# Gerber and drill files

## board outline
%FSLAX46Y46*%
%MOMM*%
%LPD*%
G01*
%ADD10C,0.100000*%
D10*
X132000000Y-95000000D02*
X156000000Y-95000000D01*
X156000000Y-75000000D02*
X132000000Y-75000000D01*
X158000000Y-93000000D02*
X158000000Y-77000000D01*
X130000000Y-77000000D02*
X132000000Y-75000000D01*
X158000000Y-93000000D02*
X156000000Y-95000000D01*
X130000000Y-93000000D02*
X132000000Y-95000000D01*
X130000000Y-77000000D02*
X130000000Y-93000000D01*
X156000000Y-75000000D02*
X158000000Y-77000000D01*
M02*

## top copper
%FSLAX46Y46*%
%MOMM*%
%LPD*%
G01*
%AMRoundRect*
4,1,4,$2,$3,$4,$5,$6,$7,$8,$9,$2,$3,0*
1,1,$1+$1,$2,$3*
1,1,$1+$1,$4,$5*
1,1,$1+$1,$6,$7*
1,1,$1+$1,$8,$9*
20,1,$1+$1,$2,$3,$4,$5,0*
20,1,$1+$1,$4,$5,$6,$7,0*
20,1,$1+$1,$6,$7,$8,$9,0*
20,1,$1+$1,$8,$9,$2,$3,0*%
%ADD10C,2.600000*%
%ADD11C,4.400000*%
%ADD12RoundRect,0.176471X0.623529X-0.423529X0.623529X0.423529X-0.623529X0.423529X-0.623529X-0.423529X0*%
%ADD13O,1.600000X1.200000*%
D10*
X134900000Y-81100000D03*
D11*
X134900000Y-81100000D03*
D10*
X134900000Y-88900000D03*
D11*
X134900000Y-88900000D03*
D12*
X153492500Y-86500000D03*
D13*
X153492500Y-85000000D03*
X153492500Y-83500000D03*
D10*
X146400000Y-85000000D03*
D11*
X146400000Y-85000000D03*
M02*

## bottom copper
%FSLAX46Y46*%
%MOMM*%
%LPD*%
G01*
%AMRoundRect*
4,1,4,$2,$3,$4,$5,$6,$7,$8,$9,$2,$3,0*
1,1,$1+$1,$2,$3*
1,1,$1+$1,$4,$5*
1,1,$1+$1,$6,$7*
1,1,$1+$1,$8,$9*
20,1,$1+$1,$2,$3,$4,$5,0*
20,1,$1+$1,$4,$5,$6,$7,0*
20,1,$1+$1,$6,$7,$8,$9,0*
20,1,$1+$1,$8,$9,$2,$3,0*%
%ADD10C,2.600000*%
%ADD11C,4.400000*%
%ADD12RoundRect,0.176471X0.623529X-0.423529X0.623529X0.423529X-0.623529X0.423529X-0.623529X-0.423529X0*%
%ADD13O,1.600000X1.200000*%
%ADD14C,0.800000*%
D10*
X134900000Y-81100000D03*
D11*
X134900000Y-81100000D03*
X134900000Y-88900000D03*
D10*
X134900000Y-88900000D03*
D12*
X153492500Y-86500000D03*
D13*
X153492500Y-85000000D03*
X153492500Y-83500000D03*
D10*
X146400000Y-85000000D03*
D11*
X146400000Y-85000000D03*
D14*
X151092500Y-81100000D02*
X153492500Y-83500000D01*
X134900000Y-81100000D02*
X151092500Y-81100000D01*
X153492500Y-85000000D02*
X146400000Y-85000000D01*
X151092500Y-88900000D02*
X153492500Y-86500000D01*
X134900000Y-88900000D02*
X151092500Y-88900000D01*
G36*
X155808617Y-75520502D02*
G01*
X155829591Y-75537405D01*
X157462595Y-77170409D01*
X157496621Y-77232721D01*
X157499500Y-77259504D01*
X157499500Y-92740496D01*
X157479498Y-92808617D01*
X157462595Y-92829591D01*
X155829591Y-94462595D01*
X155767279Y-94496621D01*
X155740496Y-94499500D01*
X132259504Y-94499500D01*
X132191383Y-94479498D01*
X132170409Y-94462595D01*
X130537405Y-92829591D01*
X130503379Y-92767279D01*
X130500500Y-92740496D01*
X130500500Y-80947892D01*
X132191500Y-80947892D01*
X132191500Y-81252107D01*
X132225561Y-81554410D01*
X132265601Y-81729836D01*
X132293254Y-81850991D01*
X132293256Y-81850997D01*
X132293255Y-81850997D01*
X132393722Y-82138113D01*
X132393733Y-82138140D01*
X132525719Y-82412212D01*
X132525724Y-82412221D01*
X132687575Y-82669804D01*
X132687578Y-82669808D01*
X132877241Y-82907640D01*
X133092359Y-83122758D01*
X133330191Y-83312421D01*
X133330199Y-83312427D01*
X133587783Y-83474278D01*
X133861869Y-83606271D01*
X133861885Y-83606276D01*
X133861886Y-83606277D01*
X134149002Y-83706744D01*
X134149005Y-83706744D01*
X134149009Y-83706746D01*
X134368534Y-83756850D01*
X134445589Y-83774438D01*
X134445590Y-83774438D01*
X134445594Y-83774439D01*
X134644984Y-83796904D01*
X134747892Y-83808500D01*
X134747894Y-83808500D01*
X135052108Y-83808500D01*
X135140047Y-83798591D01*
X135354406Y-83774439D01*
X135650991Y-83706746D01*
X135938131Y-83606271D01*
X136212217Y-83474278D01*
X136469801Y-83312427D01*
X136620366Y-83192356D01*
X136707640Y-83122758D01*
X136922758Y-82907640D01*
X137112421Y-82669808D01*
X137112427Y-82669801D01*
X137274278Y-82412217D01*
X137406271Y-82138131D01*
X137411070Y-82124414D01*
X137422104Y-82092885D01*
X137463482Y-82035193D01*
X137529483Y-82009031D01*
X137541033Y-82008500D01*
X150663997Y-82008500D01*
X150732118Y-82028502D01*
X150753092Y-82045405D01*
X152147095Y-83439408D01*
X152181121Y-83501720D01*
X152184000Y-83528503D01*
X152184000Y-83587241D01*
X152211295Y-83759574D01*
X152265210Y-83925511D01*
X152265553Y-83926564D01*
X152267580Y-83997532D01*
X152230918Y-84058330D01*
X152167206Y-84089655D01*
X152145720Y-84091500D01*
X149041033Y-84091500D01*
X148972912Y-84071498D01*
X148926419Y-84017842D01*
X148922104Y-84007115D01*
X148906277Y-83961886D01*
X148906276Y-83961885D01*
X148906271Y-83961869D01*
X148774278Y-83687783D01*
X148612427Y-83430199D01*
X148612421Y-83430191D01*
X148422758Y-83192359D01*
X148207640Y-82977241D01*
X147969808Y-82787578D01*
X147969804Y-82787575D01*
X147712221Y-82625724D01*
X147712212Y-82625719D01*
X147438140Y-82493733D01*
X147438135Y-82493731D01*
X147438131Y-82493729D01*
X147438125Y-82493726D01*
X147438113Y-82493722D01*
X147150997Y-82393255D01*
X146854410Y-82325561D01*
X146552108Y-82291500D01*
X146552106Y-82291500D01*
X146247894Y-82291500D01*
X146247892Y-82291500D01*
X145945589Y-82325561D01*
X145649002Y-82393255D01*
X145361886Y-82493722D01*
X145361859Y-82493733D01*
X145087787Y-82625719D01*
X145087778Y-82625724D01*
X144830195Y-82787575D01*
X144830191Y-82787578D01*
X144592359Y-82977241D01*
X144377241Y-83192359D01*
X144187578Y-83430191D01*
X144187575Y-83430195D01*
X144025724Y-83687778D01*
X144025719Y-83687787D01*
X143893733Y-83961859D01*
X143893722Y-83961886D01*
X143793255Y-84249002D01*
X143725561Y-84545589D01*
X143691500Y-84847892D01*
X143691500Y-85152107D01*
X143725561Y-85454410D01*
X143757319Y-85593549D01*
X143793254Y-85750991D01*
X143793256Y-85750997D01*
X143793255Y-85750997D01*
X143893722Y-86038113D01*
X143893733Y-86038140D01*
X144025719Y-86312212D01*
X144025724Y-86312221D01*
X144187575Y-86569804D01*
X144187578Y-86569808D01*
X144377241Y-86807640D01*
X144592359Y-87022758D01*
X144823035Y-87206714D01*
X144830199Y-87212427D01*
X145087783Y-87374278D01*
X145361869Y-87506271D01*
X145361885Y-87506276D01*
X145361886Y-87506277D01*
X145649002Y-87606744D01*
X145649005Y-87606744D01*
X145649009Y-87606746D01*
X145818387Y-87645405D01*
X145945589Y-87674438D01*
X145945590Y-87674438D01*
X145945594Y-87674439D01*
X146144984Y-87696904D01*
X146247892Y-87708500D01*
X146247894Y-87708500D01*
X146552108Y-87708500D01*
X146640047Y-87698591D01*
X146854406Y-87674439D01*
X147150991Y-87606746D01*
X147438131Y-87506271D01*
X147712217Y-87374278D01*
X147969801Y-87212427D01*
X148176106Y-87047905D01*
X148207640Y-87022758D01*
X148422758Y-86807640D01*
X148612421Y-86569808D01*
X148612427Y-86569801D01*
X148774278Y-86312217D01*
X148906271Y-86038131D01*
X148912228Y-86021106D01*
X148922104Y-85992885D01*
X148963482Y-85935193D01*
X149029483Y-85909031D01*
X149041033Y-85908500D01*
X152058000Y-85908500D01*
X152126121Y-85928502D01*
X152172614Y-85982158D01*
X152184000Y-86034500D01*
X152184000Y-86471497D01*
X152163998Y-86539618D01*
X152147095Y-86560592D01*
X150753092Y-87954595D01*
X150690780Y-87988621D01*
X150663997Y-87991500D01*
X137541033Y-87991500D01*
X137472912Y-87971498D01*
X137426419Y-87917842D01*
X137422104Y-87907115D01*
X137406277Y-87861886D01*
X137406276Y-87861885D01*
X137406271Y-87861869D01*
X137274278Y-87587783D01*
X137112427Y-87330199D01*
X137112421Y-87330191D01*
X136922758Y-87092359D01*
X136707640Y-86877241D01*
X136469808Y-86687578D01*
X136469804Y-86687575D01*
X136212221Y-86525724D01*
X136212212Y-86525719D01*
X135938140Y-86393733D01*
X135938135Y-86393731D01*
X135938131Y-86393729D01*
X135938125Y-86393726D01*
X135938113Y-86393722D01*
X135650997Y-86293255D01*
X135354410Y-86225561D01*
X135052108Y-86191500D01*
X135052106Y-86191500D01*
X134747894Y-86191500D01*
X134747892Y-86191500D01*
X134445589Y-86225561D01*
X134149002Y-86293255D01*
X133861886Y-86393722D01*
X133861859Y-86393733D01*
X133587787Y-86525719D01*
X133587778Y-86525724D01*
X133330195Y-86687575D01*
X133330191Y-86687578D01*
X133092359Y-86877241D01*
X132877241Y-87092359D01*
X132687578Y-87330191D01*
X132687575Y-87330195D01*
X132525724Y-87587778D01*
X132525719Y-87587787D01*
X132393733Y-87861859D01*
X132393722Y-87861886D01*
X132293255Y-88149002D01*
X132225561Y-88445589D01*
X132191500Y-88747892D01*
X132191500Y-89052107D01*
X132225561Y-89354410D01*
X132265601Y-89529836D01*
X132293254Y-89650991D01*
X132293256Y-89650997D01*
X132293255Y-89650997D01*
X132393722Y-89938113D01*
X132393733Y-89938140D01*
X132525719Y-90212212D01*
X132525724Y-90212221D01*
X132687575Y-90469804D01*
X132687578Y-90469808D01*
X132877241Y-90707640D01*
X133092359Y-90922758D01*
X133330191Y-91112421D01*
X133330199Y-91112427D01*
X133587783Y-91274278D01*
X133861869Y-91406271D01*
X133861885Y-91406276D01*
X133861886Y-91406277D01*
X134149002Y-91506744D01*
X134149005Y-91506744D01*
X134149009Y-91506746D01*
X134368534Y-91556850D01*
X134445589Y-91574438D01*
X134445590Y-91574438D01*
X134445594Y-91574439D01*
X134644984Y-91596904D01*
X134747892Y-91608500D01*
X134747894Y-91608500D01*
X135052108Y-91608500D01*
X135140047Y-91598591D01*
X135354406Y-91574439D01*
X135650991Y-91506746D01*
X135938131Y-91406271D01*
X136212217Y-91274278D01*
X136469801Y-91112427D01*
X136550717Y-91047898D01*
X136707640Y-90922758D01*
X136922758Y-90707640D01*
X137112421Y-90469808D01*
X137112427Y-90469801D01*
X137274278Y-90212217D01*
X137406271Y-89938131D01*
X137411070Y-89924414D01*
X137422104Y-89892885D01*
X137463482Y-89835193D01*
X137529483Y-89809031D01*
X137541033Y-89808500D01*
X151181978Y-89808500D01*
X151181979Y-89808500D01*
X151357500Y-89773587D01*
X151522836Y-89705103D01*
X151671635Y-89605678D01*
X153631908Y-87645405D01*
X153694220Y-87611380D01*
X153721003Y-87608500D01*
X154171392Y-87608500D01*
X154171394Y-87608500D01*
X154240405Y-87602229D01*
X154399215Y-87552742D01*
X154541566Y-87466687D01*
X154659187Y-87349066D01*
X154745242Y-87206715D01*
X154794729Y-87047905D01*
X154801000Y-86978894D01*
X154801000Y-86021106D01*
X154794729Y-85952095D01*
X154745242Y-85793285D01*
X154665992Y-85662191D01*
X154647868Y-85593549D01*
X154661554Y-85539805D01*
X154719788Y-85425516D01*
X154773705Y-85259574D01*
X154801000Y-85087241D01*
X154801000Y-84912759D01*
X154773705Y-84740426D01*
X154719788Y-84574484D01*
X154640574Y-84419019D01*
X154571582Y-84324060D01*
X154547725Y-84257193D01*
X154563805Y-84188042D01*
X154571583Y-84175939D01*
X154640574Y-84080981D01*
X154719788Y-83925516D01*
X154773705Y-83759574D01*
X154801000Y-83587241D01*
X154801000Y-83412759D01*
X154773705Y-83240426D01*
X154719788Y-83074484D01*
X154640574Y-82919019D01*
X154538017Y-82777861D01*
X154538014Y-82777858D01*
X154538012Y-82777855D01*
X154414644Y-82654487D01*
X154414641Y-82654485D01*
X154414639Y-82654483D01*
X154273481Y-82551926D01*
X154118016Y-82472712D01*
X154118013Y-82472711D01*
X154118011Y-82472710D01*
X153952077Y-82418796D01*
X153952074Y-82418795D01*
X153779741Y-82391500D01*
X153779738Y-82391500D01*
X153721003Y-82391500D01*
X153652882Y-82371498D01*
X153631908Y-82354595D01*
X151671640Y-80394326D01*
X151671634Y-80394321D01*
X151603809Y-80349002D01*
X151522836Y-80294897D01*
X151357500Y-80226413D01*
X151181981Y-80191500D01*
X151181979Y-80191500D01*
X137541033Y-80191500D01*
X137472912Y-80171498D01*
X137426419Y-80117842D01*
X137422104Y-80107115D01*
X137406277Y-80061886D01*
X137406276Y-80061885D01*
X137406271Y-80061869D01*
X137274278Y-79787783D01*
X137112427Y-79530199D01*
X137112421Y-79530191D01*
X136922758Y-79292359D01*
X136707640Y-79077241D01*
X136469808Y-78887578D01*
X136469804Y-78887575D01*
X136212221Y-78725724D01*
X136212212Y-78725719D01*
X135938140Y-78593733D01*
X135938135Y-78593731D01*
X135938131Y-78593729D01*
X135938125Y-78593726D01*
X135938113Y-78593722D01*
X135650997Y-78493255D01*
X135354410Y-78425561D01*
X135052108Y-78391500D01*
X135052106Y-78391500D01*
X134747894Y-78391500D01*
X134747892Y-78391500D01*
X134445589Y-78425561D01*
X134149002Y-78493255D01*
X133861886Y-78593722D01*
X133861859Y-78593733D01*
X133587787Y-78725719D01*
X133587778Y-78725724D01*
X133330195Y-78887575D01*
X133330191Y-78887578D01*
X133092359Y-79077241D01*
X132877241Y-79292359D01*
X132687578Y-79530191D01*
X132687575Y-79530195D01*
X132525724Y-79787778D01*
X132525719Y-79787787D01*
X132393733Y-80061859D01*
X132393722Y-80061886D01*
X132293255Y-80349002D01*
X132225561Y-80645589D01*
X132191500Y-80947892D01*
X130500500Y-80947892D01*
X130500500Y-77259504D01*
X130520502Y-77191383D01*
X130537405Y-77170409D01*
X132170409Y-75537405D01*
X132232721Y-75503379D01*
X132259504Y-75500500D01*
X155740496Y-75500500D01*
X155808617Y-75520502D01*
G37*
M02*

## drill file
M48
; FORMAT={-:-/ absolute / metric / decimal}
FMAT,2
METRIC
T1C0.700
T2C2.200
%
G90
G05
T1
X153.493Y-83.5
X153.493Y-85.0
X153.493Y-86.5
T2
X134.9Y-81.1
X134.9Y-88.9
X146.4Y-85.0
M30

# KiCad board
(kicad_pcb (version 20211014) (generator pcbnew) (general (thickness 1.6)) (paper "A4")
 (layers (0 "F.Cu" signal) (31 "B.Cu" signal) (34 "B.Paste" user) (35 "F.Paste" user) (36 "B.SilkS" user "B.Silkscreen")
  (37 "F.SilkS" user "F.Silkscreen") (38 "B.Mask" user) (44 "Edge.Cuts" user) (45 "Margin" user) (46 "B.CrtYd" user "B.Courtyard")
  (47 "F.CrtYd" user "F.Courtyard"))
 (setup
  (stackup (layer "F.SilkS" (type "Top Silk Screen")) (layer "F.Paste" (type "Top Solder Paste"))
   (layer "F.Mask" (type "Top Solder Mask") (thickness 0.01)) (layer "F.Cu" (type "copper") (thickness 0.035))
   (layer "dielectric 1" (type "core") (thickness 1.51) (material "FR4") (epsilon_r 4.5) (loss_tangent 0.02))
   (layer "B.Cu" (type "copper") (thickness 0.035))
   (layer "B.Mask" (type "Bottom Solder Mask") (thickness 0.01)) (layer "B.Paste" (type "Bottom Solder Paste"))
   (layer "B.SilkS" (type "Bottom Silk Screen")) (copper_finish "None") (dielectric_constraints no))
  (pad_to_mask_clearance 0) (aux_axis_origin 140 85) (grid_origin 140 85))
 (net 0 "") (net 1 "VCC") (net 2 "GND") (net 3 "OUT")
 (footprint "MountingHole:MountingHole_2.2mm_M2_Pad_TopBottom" (layer "F.Cu") (at 134.9 81.1)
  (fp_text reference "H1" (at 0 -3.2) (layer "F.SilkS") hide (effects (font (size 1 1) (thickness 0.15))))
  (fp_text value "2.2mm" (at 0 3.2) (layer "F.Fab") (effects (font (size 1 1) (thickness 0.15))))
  (pad "1" thru_hole circle locked (at 0 0) (size 2.6 2.6) (drill 2.2) (layers *.Cu *.Mask) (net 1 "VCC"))
  (pad "1" connect circle locked (at 0 0) (size 4.4 4.4) (layers "B.Cu" "B.Mask") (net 1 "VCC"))
  (pad "1" connect circle locked (at 0 0) (size 4.4 4.4) (layers "F.Cu" "F.Mask") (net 1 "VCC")))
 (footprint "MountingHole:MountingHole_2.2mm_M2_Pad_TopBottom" (layer "F.Cu") (at 134.9 88.9)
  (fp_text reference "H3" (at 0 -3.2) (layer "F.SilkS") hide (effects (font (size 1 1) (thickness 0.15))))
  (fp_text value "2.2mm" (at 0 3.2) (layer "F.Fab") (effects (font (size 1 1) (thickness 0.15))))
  (pad "1" connect circle locked (at 0 0) (size 4.4 4.4) (layers "B.Cu" "B.Mask") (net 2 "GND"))
  (pad "1" thru_hole circle locked (at 0 0) (size 2.6 2.6) (drill 2.2) (layers *.Cu *.Mask) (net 2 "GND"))
  (pad "1" connect circle locked (at 0 0) (size 4.4 4.4) (layers "F.Cu" "F.Mask") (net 2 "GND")))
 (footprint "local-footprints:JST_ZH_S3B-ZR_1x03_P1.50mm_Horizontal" (layer "F.Cu") (at 153.4925 86.5 90)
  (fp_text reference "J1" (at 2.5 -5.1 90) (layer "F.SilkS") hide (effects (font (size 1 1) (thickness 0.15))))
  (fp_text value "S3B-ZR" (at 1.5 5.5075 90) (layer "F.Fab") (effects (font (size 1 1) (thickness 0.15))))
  (pad "1" thru_hole roundrect (at 0 0 90) (size 1.2 1.6) (drill 0.7) (layers *.Cu *.Mask) (roundrect_rratio 0.1470591667) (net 2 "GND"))
  (pad "2" thru_hole oval (at 1.5 0 90) (size 1.2 1.6) (drill 0.7) (layers *.Cu *.Mask) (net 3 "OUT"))
  (pad "3" thru_hole oval (at 3 0 90) (size 1.2 1.6) (drill 0.7) (layers *.Cu *.Mask) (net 1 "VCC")))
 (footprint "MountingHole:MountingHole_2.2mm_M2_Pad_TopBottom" (layer "F.Cu") (at 146.4 85)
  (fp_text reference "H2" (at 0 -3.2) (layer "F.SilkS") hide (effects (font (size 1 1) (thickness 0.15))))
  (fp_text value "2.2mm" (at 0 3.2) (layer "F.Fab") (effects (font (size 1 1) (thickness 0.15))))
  (pad "1" thru_hole circle locked (at 0 0) (size 2.6 2.6) (drill 2.2) (layers *.Cu *.Mask) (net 3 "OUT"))
  (pad "1" connect circle locked (at 0 0) (size 4.4 4.4) (layers "B.Cu" "B.Mask") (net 3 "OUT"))
  (pad "1" connect circle locked (at 0 0) (size 4.4 4.4) (layers "F.Cu" "F.Mask") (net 3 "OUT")))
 (gr_line (start 132 95) (end 156 95) (layer "Edge.Cuts") (width 0.1))
 (gr_line (start 156 75) (end 132 75) (layer "Edge.Cuts") (width 0.1))
 (gr_line (start 158 93) (end 158 77) (layer "Edge.Cuts") (width 0.1))
 (gr_line (start 130 77) (end 132 75) (layer "Edge.Cuts") (width 0.1))
 (gr_line (start 158 93) (end 156 95) (layer "Edge.Cuts") (width 0.1))
 (gr_line (start 130 93) (end 132 95) (layer "Edge.Cuts") (width 0.1))
 (gr_line (start 130 77) (end 130 93) (layer "Edge.Cuts") (width 0.1))
 (gr_line (start 156 75) (end 158 77) (layer "Edge.Cuts") (width 0.1))
 (segment (start 151.0925 81.1) (end 153.4925 83.5) (width 0.8) (layer "B.Cu") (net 1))
 (segment (start 134.9 81.1) (end 151.0925 81.1) (width 0.8) (layer "B.Cu") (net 1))
 (segment (start 153.4925 85) (end 146.4 85) (width 0.8) (layer "B.Cu") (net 3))
 (segment (start 151.0925 88.9) (end 153.4925 86.5) (width 0.8) (layer "B.Cu") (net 2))
 (segment (start 134.9 88.9) (end 151.0925 88.9) (width 0.8) (layer "B.Cu") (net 2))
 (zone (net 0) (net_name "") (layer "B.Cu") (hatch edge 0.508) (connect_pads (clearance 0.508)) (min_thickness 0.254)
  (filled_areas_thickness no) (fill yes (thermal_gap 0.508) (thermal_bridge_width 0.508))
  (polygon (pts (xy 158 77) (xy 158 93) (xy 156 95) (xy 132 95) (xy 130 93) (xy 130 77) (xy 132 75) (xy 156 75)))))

